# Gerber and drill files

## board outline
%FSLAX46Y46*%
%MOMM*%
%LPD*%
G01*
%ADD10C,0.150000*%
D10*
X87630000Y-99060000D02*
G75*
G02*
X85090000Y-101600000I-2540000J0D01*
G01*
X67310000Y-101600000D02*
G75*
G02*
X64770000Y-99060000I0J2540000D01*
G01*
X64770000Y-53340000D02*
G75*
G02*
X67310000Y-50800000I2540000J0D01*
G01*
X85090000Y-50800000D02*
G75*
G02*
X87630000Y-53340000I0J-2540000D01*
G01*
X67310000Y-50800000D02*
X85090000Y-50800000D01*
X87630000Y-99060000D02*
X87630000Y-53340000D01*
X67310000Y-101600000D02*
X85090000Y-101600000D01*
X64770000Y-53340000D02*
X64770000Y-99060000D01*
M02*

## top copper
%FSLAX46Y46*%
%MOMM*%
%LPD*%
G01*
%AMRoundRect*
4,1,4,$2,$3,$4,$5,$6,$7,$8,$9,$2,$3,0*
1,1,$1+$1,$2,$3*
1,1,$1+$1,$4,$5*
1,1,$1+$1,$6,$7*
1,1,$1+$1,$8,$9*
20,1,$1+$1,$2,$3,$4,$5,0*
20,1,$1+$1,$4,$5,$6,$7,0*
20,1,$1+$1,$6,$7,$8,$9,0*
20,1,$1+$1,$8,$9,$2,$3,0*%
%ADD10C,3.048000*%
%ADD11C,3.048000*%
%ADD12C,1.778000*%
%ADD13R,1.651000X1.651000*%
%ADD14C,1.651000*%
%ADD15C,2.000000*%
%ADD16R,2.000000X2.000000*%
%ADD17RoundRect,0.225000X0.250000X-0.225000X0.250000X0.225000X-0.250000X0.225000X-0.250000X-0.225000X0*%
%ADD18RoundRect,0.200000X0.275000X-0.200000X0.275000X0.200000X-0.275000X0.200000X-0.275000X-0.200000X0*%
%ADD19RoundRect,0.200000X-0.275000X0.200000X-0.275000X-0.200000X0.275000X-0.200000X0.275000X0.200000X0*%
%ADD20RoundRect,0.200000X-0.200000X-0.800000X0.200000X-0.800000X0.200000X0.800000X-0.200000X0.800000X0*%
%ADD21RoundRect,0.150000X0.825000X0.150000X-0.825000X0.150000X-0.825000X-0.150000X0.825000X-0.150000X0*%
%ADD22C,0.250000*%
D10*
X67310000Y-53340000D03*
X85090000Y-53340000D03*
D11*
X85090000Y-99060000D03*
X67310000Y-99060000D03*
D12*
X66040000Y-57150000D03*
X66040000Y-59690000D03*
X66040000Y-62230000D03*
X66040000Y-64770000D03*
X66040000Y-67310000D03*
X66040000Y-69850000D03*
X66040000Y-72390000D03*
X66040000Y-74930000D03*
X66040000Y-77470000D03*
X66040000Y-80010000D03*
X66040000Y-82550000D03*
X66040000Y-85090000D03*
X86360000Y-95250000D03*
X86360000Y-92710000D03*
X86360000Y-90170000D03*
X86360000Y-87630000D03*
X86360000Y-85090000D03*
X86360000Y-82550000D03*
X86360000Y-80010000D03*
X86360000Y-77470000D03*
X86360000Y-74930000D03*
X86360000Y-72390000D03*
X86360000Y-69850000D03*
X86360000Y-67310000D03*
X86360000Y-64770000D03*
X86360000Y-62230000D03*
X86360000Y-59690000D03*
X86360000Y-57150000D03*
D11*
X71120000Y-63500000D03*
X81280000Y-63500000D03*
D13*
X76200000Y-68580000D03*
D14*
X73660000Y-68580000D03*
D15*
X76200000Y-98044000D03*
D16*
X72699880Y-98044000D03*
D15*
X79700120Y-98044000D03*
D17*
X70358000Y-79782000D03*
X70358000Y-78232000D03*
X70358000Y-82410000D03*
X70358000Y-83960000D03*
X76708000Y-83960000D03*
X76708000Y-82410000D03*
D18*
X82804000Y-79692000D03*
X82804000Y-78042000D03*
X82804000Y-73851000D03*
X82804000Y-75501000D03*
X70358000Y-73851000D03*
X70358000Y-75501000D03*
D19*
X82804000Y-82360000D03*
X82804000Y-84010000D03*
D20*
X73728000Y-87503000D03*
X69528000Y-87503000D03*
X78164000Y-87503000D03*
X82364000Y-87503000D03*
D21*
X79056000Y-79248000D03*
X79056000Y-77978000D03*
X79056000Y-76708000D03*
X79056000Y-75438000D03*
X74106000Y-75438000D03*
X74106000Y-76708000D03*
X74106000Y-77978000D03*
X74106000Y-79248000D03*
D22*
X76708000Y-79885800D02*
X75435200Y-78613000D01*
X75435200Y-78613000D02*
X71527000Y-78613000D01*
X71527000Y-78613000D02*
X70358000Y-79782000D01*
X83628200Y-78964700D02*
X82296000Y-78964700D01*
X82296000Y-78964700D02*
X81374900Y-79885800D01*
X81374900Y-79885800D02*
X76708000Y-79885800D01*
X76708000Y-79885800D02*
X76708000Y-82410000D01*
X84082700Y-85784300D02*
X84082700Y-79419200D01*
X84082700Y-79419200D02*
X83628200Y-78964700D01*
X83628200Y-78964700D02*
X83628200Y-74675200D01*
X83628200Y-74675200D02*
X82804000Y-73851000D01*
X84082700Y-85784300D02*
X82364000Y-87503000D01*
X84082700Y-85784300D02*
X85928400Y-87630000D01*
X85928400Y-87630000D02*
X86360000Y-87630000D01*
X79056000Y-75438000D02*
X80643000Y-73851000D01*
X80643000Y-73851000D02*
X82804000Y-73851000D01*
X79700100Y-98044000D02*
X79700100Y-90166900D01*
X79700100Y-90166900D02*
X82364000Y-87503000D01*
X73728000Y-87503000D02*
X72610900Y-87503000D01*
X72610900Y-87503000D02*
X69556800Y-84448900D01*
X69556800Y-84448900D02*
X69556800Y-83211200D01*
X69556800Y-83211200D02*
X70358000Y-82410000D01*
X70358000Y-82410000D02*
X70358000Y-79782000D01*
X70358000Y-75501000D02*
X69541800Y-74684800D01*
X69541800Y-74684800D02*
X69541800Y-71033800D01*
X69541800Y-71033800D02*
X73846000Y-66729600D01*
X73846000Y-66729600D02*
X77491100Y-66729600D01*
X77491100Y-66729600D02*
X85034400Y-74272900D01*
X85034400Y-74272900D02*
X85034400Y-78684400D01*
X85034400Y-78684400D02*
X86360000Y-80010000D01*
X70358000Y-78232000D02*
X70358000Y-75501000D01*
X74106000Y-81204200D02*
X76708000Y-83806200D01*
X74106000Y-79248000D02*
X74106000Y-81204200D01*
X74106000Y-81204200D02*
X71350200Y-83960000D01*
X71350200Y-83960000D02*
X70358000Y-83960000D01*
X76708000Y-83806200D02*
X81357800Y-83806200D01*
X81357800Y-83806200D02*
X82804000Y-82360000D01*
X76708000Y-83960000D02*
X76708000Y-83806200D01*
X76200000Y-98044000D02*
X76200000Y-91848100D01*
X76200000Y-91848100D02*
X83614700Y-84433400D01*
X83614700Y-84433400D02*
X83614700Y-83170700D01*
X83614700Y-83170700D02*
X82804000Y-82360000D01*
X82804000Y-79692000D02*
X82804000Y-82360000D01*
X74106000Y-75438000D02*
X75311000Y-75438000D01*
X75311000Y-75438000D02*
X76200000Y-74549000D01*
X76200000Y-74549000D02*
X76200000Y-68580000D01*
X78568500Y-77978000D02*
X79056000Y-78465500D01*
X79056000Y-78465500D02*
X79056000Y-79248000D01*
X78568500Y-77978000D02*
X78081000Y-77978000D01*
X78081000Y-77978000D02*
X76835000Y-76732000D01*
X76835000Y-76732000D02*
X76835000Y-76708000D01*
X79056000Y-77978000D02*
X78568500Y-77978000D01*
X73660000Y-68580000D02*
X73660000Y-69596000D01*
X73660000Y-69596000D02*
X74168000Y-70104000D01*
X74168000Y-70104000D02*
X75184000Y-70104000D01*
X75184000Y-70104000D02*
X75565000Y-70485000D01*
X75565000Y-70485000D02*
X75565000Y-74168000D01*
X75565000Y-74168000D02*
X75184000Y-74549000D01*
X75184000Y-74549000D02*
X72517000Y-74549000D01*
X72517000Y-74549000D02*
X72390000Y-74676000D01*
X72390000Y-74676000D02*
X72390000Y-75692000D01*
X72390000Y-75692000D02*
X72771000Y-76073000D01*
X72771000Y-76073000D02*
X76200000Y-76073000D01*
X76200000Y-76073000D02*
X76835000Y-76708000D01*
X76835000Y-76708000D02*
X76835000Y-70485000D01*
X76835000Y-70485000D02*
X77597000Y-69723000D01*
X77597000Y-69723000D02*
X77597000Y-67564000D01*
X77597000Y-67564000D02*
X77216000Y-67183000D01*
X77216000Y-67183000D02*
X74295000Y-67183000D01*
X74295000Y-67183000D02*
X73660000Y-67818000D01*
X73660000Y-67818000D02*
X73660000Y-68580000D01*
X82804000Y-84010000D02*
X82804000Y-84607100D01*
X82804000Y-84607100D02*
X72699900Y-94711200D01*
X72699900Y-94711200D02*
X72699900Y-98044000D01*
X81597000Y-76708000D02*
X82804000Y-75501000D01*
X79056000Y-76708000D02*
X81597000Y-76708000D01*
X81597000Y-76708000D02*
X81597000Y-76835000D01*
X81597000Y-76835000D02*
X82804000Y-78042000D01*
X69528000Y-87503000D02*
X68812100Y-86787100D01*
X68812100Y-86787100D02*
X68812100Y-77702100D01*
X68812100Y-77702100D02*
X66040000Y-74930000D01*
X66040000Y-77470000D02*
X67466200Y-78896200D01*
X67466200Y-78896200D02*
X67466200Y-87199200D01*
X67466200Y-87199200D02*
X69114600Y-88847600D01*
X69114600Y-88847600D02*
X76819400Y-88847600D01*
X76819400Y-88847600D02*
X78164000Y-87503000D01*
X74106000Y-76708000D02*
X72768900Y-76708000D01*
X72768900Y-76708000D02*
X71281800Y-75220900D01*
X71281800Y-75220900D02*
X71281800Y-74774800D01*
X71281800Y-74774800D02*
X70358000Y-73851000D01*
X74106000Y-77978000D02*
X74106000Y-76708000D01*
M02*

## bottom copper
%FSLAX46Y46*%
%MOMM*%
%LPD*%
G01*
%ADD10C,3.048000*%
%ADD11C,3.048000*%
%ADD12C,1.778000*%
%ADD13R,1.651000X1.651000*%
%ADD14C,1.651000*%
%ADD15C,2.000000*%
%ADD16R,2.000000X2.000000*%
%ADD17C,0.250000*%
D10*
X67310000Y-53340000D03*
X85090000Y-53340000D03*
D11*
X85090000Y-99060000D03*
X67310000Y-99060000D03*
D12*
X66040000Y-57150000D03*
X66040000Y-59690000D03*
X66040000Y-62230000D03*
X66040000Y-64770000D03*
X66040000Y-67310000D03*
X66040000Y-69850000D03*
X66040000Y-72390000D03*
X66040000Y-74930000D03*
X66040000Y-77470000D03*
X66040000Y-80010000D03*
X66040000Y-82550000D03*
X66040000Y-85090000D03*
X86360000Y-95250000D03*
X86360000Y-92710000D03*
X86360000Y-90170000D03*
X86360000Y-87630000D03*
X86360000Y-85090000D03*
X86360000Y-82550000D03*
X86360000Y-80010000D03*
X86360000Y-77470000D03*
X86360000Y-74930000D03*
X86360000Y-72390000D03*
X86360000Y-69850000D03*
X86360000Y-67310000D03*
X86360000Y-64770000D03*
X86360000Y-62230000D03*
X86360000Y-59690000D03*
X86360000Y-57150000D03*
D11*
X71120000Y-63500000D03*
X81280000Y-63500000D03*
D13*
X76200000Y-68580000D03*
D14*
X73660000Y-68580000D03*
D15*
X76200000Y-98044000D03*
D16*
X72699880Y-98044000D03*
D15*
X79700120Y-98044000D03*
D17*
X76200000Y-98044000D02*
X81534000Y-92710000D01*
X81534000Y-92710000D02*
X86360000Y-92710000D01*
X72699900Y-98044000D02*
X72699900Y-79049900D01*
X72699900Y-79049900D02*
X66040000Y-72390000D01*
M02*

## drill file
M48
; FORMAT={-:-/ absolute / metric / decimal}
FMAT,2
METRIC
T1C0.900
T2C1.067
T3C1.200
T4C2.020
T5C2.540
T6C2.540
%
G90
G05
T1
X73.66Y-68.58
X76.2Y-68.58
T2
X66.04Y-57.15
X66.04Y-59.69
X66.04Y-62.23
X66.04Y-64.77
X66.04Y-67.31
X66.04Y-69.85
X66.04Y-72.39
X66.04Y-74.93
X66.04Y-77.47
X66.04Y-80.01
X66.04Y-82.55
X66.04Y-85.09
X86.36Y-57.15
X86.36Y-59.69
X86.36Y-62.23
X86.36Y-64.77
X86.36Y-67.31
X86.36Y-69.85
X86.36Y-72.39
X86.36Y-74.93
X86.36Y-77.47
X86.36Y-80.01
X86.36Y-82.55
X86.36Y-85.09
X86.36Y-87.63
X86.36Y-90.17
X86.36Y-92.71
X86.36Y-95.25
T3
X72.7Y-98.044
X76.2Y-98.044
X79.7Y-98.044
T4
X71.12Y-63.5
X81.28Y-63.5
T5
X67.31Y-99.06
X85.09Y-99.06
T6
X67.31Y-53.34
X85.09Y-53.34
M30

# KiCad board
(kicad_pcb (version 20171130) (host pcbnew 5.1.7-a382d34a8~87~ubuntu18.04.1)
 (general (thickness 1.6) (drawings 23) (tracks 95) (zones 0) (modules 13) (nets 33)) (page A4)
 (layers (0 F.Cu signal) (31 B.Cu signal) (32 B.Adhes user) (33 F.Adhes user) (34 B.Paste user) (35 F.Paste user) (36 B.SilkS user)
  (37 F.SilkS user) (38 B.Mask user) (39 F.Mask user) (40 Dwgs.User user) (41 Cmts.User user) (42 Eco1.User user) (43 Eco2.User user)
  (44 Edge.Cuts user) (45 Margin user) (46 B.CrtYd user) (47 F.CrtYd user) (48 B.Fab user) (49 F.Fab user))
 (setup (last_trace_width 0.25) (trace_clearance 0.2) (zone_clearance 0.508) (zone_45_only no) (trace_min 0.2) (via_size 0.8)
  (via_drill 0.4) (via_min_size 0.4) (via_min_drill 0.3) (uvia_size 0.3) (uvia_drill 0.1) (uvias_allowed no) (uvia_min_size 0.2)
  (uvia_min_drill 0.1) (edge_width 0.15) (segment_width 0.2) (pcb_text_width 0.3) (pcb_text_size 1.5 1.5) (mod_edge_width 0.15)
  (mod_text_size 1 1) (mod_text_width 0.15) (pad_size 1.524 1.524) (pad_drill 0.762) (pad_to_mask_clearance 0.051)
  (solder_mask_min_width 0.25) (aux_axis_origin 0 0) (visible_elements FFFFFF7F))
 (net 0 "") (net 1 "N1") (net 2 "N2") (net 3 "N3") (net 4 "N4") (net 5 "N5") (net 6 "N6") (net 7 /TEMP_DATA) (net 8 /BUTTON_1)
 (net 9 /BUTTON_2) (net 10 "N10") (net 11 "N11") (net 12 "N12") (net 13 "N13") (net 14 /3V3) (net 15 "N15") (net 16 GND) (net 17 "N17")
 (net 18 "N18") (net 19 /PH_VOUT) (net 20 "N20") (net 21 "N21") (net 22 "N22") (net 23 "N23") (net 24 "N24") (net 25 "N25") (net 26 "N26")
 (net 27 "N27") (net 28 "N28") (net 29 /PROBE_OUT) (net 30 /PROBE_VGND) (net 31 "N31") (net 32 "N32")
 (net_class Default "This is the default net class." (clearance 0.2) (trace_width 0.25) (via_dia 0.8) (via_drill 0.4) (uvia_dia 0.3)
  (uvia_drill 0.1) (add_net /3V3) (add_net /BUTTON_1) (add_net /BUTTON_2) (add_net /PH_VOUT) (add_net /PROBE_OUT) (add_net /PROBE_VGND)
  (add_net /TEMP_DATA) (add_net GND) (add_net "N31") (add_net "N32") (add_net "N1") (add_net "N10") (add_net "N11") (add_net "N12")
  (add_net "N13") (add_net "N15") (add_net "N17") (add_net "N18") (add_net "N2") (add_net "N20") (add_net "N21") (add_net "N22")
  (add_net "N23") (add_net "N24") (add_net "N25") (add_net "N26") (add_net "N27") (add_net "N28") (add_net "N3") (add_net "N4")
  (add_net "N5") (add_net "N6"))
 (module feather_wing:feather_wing (layer F.Cu) (at 76.2 76.2)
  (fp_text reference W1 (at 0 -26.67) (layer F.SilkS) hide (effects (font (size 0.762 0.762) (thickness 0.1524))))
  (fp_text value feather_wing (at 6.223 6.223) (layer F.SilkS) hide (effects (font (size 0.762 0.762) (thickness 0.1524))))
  (pad "" np_thru_hole circle (at -8.89 -22.86) (size 3.048 3.048) (drill 2.54) (layers *.Cu *.Mask))
  (pad "" np_thru_hole circle (at 8.89 -22.86) (size 3.048 3.048) (drill 2.54) (layers *.Cu *.Mask))
  (pad "" thru_hole circle (at 8.89 22.86) (size 3.048 3.048) (drill 2.54) (layers *.Cu *.Mask))
  (pad "" thru_hole circle (at -8.89 22.86) (size 3.048 3.048) (drill 2.54) (layers *.Cu *.Mask))
  (pad 1 thru_hole circle (at -10.16 -19.05) (size 1.778 1.778) (drill 1.0668) (layers *.Cu *.Mask) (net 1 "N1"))
  (pad 2 thru_hole circle (at -10.16 -16.51) (size 1.778 1.778) (drill 1.0668) (layers *.Cu *.Mask) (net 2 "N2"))
  (pad 3 thru_hole circle (at -10.16 -13.97) (size 1.778 1.778) (drill 1.0668) (layers *.Cu *.Mask) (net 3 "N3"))
  (pad 4 thru_hole circle (at -10.16 -11.43) (size 1.778 1.778) (drill 1.0668) (layers *.Cu *.Mask) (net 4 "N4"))
  (pad 5 thru_hole circle (at -10.16 -8.89) (size 1.778 1.778) (drill 1.0668) (layers *.Cu *.Mask) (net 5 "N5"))
  (pad 6 thru_hole circle (at -10.16 -6.35) (size 1.778 1.778) (drill 1.0668) (layers *.Cu *.Mask) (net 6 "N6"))
  (pad 7 thru_hole circle (at -10.16 -3.81) (size 1.778 1.778) (drill 1.0668) (layers *.Cu *.Mask) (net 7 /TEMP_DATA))
  (pad 8 thru_hole circle (at -10.16 -1.27) (size 1.778 1.778) (drill 1.0668) (layers *.Cu *.Mask) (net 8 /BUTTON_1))
  (pad 9 thru_hole circle (at -10.16 1.27) (size 1.778 1.778) (drill 1.0668) (layers *.Cu *.Mask) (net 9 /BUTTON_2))
  (pad 10 thru_hole circle (at -10.16 3.81) (size 1.778 1.778) (drill 1.0668) (layers *.Cu *.Mask) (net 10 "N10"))
  (pad 11 thru_hole circle (at -10.16 6.35) (size 1.778 1.778) (drill 1.0668) (layers *.Cu *.Mask) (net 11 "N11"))
  (pad 12 thru_hole circle (at -10.16 8.89) (size 1.778 1.778) (drill 1.0668) (layers *.Cu *.Mask) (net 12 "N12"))
  (pad 13 thru_hole circle (at 10.16 19.05) (size 1.778 1.778) (drill 1.0668) (layers *.Cu *.Mask) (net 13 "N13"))
  (pad 14 thru_hole circle (at 10.16 16.51) (size 1.778 1.778) (drill 1.0668) (layers *.Cu *.Mask) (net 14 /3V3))
  (pad 15 thru_hole circle (at 10.16 13.97) (size 1.778 1.778) (drill 1.0668) (layers *.Cu *.Mask) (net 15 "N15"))
  (pad 16 thru_hole circle (at 10.16 11.43) (size 1.778 1.778) (drill 1.0668) (layers *.Cu *.Mask) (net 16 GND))
  (pad 17 thru_hole circle (at 10.16 8.89) (size 1.778 1.778) (drill 1.0668) (layers *.Cu *.Mask) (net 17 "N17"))
  (pad 18 thru_hole circle (at 10.16 6.35) (size 1.778 1.778) (drill 1.0668) (layers *.Cu *.Mask) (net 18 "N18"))
  (pad 19 thru_hole circle (at 10.16 3.81) (size 1.778 1.778) (drill 1.0668) (layers *.Cu *.Mask) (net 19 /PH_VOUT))
  (pad 20 thru_hole circle (at 10.16 1.27) (size 1.778 1.778) (drill 1.0668) (layers *.Cu *.Mask) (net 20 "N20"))
  (pad 21 thru_hole circle (at 10.16 -1.27) (size 1.778 1.778) (drill 1.0668) (layers *.Cu *.Mask) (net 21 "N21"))
  (pad 22 thru_hole circle (at 10.16 -3.81) (size 1.778 1.778) (drill 1.0668) (layers *.Cu *.Mask) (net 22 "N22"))
  (pad 23 thru_hole circle (at 10.16 -6.35) (size 1.778 1.778) (drill 1.0668) (layers *.Cu *.Mask) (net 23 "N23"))
  (pad 24 thru_hole circle (at 10.16 -8.89) (size 1.778 1.778) (drill 1.0668) (layers *.Cu *.Mask) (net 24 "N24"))
  (pad 25 thru_hole circle (at 10.16 -11.43) (size 1.778 1.778) (drill 1.0668) (layers *.Cu *.Mask) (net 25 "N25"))
  (pad 26 thru_hole circle (at 10.16 -13.97) (size 1.778 1.778) (drill 1.0668) (layers *.Cu *.Mask) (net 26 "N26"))
  (pad 27 thru_hole circle (at 10.16 -16.51) (size 1.778 1.778) (drill 1.0668) (layers *.Cu *.Mask) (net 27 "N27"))
  (pad 28 thru_hole circle (at 10.16 -19.05) (size 1.778 1.778) (drill 1.0668) (layers *.Cu *.Mask) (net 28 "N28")))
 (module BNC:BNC (layer F.Cu) (at 76.2 63.5)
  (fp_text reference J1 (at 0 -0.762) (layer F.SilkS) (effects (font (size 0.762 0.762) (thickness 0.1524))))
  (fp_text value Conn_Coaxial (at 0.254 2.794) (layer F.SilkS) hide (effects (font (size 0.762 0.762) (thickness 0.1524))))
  (pad "" thru_hole circle (at -5.08 0) (size 3.048 3.048) (drill 2.02) (layers *.Cu *.Mask))
  (pad "" thru_hole circle (at 5.08 0) (size 3.048 3.048) (drill 2.02) (layers *.Cu *.Mask))
  (pad 1 thru_hole rect (at 0 5.08) (size 1.651 1.651) (drill 0.9) (layers *.Cu *.Mask) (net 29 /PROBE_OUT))
  (pad 2 thru_hole circle (at -2.54 5.08) (size 1.651 1.651) (drill 0.9) (layers *.Cu *.Mask) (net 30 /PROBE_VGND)))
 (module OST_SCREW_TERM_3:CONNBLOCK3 (layer F.Cu) (at 76.2 98.044)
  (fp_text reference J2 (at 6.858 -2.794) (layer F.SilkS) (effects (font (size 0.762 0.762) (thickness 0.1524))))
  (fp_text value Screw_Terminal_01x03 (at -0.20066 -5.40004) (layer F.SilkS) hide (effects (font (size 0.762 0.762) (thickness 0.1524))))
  (pad 2 thru_hole circle (at 0 0) (size 2 2) (drill 1.2) (layers *.Cu *.Mask) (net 14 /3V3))
  (pad 1 thru_hole rect (at -3.50012 0) (size 2 2) (drill 1.2) (layers *.Cu *.Mask) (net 7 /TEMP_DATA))
  (pad 3 thru_hole circle (at 3.50012 0) (size 2 2) (drill 1.2) (layers *.Cu *.Mask) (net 16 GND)))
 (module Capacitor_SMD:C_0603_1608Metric (layer F.Cu) (at 70.358 79.007 90)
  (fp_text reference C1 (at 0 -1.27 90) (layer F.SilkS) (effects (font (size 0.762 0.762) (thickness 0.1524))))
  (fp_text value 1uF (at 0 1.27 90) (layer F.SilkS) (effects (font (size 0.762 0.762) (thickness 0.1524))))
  (pad 1 smd roundrect (at -0.775 0 90) (size 0.9 0.95) (layers F.Cu F.Paste F.Mask) (roundrect_rratio 0.25) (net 16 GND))
  (pad 2 smd roundrect (at 0.775 0 90) (size 0.9 0.95) (layers F.Cu F.Paste F.Mask) (roundrect_rratio 0.25) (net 19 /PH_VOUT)))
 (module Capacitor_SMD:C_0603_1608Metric (layer F.Cu) (at 70.358 83.185 90)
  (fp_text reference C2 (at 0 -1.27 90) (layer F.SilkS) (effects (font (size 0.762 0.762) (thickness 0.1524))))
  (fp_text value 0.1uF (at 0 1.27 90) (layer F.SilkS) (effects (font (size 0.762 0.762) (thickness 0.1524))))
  (pad 2 smd roundrect (at 0.775 0 90) (size 0.9 0.95) (layers F.Cu F.Paste F.Mask) (roundrect_rratio 0.25) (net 16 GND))
  (pad 1 smd roundrect (at -0.775 0 90) (size 0.9 0.95) (layers F.Cu F.Paste F.Mask) (roundrect_rratio 0.25) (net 14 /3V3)))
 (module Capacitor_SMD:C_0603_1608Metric (layer F.Cu) (at 76.708 83.185 90)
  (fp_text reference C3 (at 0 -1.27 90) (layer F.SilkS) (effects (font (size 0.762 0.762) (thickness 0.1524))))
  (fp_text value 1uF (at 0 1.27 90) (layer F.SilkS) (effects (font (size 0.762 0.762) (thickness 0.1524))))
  (pad 1 smd roundrect (at -0.775 0 90) (size 0.9 0.95) (layers F.Cu F.Paste F.Mask) (roundrect_rratio 0.25) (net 14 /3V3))
  (pad 2 smd roundrect (at 0.775 0 90) (size 0.9 0.95) (layers F.Cu F.Paste F.Mask) (roundrect_rratio 0.25) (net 16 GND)))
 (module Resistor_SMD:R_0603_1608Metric (layer F.Cu) (at 82.804 78.867 90)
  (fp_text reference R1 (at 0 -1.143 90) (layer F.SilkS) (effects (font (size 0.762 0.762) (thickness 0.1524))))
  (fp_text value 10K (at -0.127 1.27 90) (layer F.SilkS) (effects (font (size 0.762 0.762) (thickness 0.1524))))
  (pad 1 smd roundrect (at -0.825 0 90) (size 0.8 0.95) (layers F.Cu F.Paste F.Mask) (roundrect_rratio 0.25) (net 14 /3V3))
  (pad 2 smd roundrect (at 0.825 0 90) (size 0.8 0.95) (layers F.Cu F.Paste F.Mask) (roundrect_rratio 0.25) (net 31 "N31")))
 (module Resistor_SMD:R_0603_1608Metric (layer F.Cu) (at 82.804 74.676 90)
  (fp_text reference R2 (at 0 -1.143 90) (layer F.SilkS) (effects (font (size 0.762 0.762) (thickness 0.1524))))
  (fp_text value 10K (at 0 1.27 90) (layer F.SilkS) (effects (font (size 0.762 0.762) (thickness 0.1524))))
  (pad 2 smd roundrect (at 0.825 0 90) (size 0.8 0.95) (layers F.Cu F.Paste F.Mask) (roundrect_rratio 0.25) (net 16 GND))
  (pad 1 smd roundrect (at -0.825 0 90) (size 0.8 0.95) (layers F.Cu F.Paste F.Mask) (roundrect_rratio 0.25) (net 31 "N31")))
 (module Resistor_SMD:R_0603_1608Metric (layer F.Cu) (at 70.358 74.676 90)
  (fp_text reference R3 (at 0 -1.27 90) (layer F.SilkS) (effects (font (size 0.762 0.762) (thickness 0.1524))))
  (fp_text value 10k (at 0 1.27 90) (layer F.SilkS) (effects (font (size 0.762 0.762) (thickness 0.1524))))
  (pad 2 smd roundrect (at 0.825 0 90) (size 0.8 0.95) (layers F.Cu F.Paste F.Mask) (roundrect_rratio 0.25) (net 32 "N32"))
  (pad 1 smd roundrect (at -0.825 0 90) (size 0.8 0.95) (layers F.Cu F.Paste F.Mask) (roundrect_rratio 0.25) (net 19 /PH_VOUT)))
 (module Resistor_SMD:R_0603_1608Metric (layer F.Cu) (at 82.804 83.185 270)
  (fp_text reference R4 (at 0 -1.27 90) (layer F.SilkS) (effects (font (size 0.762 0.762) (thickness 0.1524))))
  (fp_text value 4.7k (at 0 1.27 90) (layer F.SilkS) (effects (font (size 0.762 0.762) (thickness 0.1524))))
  (pad 1 smd roundrect (at -0.825 0 270) (size 0.8 0.95) (layers F.Cu F.Paste F.Mask) (roundrect_rratio 0.25) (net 14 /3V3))
  (pad 2 smd roundrect (at 0.825 0 270) (size 0.8 0.95) (layers F.Cu F.Paste F.Mask) (roundrect_rratio 0.25) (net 7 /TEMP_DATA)))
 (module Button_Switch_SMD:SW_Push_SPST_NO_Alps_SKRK (layer F.Cu) (at 71.628 87.503)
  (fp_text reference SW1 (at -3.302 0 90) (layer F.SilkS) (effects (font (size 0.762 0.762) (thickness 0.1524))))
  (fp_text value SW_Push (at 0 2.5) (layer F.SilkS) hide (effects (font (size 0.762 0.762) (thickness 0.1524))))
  (pad 2 smd roundrect (at 2.1 0) (size 0.8 2) (layers F.Cu F.Paste F.Mask) (roundrect_rratio 0.25) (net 16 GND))
  (pad 1 smd roundrect (at -2.1 0) (size 0.8 2) (layers F.Cu F.Paste F.Mask) (roundrect_rratio 0.25) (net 8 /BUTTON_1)))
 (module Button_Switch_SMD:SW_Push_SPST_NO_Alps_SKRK (layer F.Cu) (at 80.264 87.503)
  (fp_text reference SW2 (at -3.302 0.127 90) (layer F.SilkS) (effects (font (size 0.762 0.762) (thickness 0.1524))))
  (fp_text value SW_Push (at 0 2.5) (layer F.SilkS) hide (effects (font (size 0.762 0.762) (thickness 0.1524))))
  (pad 1 smd roundrect (at -2.1 0) (size 0.8 2) (layers F.Cu F.Paste F.Mask) (roundrect_rratio 0.25) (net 9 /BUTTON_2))
  (pad 2 smd roundrect (at 2.1 0) (size 0.8 2) (layers F.Cu F.Paste F.Mask) (roundrect_rratio 0.25) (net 16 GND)))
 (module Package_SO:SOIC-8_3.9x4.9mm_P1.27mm (layer F.Cu) (at 76.581 77.343 180)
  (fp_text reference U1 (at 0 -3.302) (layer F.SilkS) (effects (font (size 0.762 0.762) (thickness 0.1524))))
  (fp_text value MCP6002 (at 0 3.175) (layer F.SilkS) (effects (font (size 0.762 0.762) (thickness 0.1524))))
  (pad 1 smd roundrect (at -2.475 -1.905 180) (size 1.95 0.6) (layers F.Cu F.Paste F.Mask) (roundrect_rratio 0.25) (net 30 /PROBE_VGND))
  (pad 2 smd roundrect (at -2.475 -0.635 180) (size 1.95 0.6) (layers F.Cu F.Paste F.Mask) (roundrect_rratio 0.25) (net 30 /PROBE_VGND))
  (pad 3 smd roundrect (at -2.475 0.635 180) (size 1.95 0.6) (layers F.Cu F.Paste F.Mask) (roundrect_rratio 0.25) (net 31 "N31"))
  (pad 4 smd roundrect (at -2.475 1.905 180) (size 1.95 0.6) (layers F.Cu F.Paste F.Mask) (roundrect_rratio 0.25) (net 16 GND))
  (pad 5 smd roundrect (at 2.475 1.905 180) (size 1.95 0.6) (layers F.Cu F.Paste F.Mask) (roundrect_rratio 0.25) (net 29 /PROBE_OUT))
  (pad 6 smd roundrect (at 2.475 0.635 180) (size 1.95 0.6) (layers F.Cu F.Paste F.Mask) (roundrect_rratio 0.25) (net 32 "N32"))
  (pad 7 smd roundrect (at 2.475 -0.635 180) (size 1.95 0.6) (layers F.Cu F.Paste F.Mask) (roundrect_rratio 0.25) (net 32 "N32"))
  (pad 8 smd roundrect (at 2.475 -1.905 180) (size 1.95 0.6) (layers F.Cu F.Paste F.Mask) (roundrect_rratio 0.25) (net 14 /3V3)))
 (gr_arc (start 85.09 99.06) (end 85.09 101.6) (angle -90) (layer Edge.Cuts) (width 0.15))
 (gr_arc (start 67.31 99.06) (end 64.77 99.06) (angle -90) (layer Edge.Cuts) (width 0.15))
 (gr_arc (start 67.31 53.34) (end 67.31 50.8) (angle -90) (layer Edge.Cuts) (width 0.15))
 (gr_arc (start 85.09 53.34) (end 87.63 53.34) (angle -90) (layer Edge.Cuts) (width 0.15))
 (gr_line (start 67.31 50.8) (end 85.09 50.8) (layer Edge.Cuts) (width 0.15))
 (gr_line (start 87.63 99.06) (end 87.63 53.34) (layer Edge.Cuts) (width 0.15))
 (gr_line (start 67.31 101.6) (end 85.09 101.6) (layer Edge.Cuts) (width 0.15))
 (gr_line (start 64.77 53.34) (end 64.77 99.06) (layer Edge.Cuts) (width 0.15))
 (segment (start 76.708 79.8858) (end 75.4352 78.613) (width 0.25) (layer F.Cu) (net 16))
 (segment (start 75.4352 78.613) (end 71.527 78.613) (width 0.25) (layer F.Cu) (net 16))
 (segment (start 71.527 78.613) (end 70.358 79.782) (width 0.25) (layer F.Cu) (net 16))
 (segment (start 83.6282 78.9647) (end 82.296 78.9647) (width 0.25) (layer F.Cu) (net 16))
 (segment (start 82.296 78.9647) (end 81.3749 79.8858) (width 0.25) (layer F.Cu) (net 16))
 (segment (start 81.3749 79.8858) (end 76.708 79.8858) (width 0.25) (layer F.Cu) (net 16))
 (segment (start 76.708 79.8858) (end 76.708 82.41) (width 0.25) (layer F.Cu) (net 16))
 (segment (start 84.0827 85.7843) (end 84.0827 79.4192) (width 0.25) (layer F.Cu) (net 16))
 (segment (start 84.0827 79.4192) (end 83.6282 78.9647) (width 0.25) (layer F.Cu) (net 16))
 (segment (start 83.6282 78.9647) (end 83.6282 74.6752) (width 0.25) (layer F.Cu) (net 16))
 (segment (start 83.6282 74.6752) (end 82.804 73.851) (width 0.25) (layer F.Cu) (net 16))
 (segment (start 84.0827 85.7843) (end 82.364 87.503) (width 0.25) (layer F.Cu) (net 16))
 (segment (start 84.0827 85.7843) (end 85.9284 87.63) (width 0.25) (layer F.Cu) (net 16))
 (segment (start 85.9284 87.63) (end 86.36 87.63) (width 0.25) (layer F.Cu) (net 16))
 (segment (start 79.056 75.438) (end 80.643 73.851) (width 0.25) (layer F.Cu) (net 16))
 (segment (start 80.643 73.851) (end 82.804 73.851) (width 0.25) (layer F.Cu) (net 16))
 (segment (start 79.7001 98.044) (end 79.7001 90.1669) (width 0.25) (layer F.Cu) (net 16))
 (segment (start 79.7001 90.1669) (end 82.364 87.503) (width 0.25) (layer F.Cu) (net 16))
 (segment (start 73.728 87.503) (end 72.6109 87.503) (width 0.25) (layer F.Cu) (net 16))
 (segment (start 72.6109 87.503) (end 69.5568 84.4489) (width 0.25) (layer F.Cu) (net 16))
 (segment (start 69.5568 84.4489) (end 69.5568 83.2112) (width 0.25) (layer F.Cu) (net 16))
 (segment (start 69.5568 83.2112) (end 70.358 82.41) (width 0.25) (layer F.Cu) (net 16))
 (segment (start 70.358 82.41) (end 70.358 79.782) (width 0.25) (layer F.Cu) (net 16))
 (segment (start 70.358 75.501) (end 69.5418 74.6848) (width 0.25) (layer F.Cu) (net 19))
 (segment (start 69.5418 74.6848) (end 69.5418 71.0338) (width 0.25) (layer F.Cu) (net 19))
 (segment (start 69.5418 71.0338) (end 73.846 66.7296) (width 0.25) (layer F.Cu) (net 19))
 (segment (start 73.846 66.7296) (end 77.4911 66.7296) (width 0.25) (layer F.Cu) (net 19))
 (segment (start 77.4911 66.7296) (end 85.0344 74.2729) (width 0.25) (layer F.Cu) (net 19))
 (segment (start 85.0344 74.2729) (end 85.0344 78.6844) (width 0.25) (layer F.Cu) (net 19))
 (segment (start 85.0344 78.6844) (end 86.36 80.01) (width 0.25) (layer F.Cu) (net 19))
 (segment (start 70.358 78.232) (end 70.358 75.501) (width 0.25) (layer F.Cu) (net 19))
 (segment (start 74.106 81.2042) (end 76.708 83.8062) (width 0.25) (layer F.Cu) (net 14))
 (segment (start 74.106 79.248) (end 74.106 81.2042) (width 0.25) (layer F.Cu) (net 14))
 (segment (start 74.106 81.2042) (end 71.3502 83.96) (width 0.25) (layer F.Cu) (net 14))
 (segment (start 71.3502 83.96) (end 70.358 83.96) (width 0.25) (layer F.Cu) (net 14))
 (segment (start 76.708 83.8062) (end 81.3578 83.8062) (width 0.25) (layer F.Cu) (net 14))
 (segment (start 81.3578 83.8062) (end 82.804 82.36) (width 0.25) (layer F.Cu) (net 14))
 (segment (start 76.708 83.96) (end 76.708 83.8062) (width 0.25) (layer F.Cu) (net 14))
 (segment (start 76.2 98.044) (end 76.2 91.8481) (width 0.25) (layer F.Cu) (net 14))
 (segment (start 76.2 91.8481) (end 83.6147 84.4334) (width 0.25) (layer F.Cu) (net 14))
 (segment (start 83.6147 84.4334) (end 83.6147 83.1707) (width 0.25) (layer F.Cu) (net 14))
 (segment (start 83.6147 83.1707) (end 82.804 82.36) (width 0.25) (layer F.Cu) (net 14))
 (segment (start 82.804 79.692) (end 82.804 82.36) (width 0.25) (layer F.Cu) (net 14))
 (segment (start 76.2 98.044) (end 81.534 92.71) (width 0.25) (layer B.Cu) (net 14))
 (segment (start 81.534 92.71) (end 86.36 92.71) (width 0.25) (layer B.Cu) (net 14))
 (segment (start 74.106 75.438) (end 75.311 75.438) (width 0.25) (layer F.Cu) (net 29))
 (segment (start 75.311 75.438) (end 76.2 74.549) (width 0.25) (layer F.Cu) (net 29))
 (segment (start 76.2 74.549) (end 76.2 68.58) (width 0.25) (layer F.Cu) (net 29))
 (segment (start 78.5685 77.978) (end 79.056 78.4655) (width 0.25) (layer F.Cu) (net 30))
 (segment (start 79.056 78.4655) (end 79.056 79.248) (width 0.25) (layer F.Cu) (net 30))
 (segment (start 78.5685 77.978) (end 78.081 77.978) (width 0.25) (layer F.Cu) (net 30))
 (segment (start 78.081 77.978) (end 76.835 76.732) (width 0.25) (layer F.Cu) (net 30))
 (segment (start 76.835 76.732) (end 76.835 76.708) (width 0.25) (layer F.Cu) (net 30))
 (segment (start 79.056 77.978) (end 78.5685 77.978) (width 0.25) (layer F.Cu) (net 30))
 (segment (start 73.66 68.58) (end 73.66 69.596) (width 0.25) (layer F.Cu) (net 30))
 (segment (start 73.66 69.596) (end 74.168 70.104) (width 0.25) (layer F.Cu) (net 30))
 (segment (start 74.168 70.104) (end 75.184 70.104) (width 0.25) (layer F.Cu) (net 30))
 (segment (start 75.184 70.104) (end 75.565 70.485) (width 0.25) (layer F.Cu) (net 30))
 (segment (start 75.565 70.485) (end 75.565 74.168) (width 0.25) (layer F.Cu) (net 30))
 (segment (start 75.565 74.168) (end 75.184 74.549) (width 0.25) (layer F.Cu) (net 30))
 (segment (start 75.184 74.549) (end 72.517 74.549) (width 0.25) (layer F.Cu) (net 30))
 (segment (start 72.517 74.549) (end 72.39 74.676) (width 0.25) (layer F.Cu) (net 30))
 (segment (start 72.39 74.676) (end 72.39 75.692) (width 0.25) (layer F.Cu) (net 30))
 (segment (start 72.39 75.692) (end 72.771 76.073) (width 0.25) (layer F.Cu) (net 30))
 (segment (start 72.771 76.073) (end 76.2 76.073) (width 0.25) (layer F.Cu) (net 30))
 (segment (start 76.2 76.073) (end 76.835 76.708) (width 0.25) (layer F.Cu) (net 30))
 (segment (start 76.835 76.708) (end 76.835 70.485) (width 0.25) (layer F.Cu) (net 30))
 (segment (start 76.835 70.485) (end 77.597 69.723) (width 0.25) (layer F.Cu) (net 30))
 (segment (start 77.597 69.723) (end 77.597 67.564) (width 0.25) (layer F.Cu) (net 30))
 (segment (start 77.597 67.564) (end 77.216 67.183) (width 0.25) (layer F.Cu) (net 30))
 (segment (start 77.216 67.183) (end 74.295 67.183) (width 0.25) (layer F.Cu) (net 30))
 (segment (start 74.295 67.183) (end 73.66 67.818) (width 0.25) (layer F.Cu) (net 30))
 (segment (start 73.66 67.818) (end 73.66 68.58) (width 0.25) (layer F.Cu) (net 30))
 (segment (start 72.6999 98.044) (end 72.6999 79.0499) (width 0.25) (layer B.Cu) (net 7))
 (segment (start 72.6999 79.0499) (end 66.04 72.39) (width 0.25) (layer B.Cu) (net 7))
 (segment (start 82.804 84.01) (end 82.804 84.6071) (width 0.25) (layer F.Cu) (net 7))
 (segment (start 82.804 84.6071) (end 72.6999 94.7112) (width 0.25) (layer F.Cu) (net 7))
 (segment (start 72.6999 94.7112) (end 72.6999 98.044) (width 0.25) (layer F.Cu) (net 7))
 (segment (start 81.597 76.708) (end 82.804 75.501) (width 0.25) (layer F.Cu) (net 31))
 (segment (start 79.056 76.708) (end 81.597 76.708) (width 0.25) (layer F.Cu) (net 31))
 (segment (start 81.597 76.708) (end 81.597 76.835) (width 0.25) (layer F.Cu) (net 31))
 (segment (start 81.597 76.835) (end 82.804 78.042) (width 0.25) (layer F.Cu) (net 31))
 (segment (start 69.528 87.503) (end 68.8121 86.7871) (width 0.25) (layer F.Cu) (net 8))
 (segment (start 68.8121 86.7871) (end 68.8121 77.7021) (width 0.25) (layer F.Cu) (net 8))
 (segment (start 68.8121 77.7021) (end 66.04 74.93) (width 0.25) (layer F.Cu) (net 8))
 (segment (start 66.04 77.47) (end 67.4662 78.8962) (width 0.25) (layer F.Cu) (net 9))
 (segment (start 67.4662 78.8962) (end 67.4662 87.1992) (width 0.25) (layer F.Cu) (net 9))
 (segment (start 67.4662 87.1992) (end 69.1146 88.8476) (width 0.25) (layer F.Cu) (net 9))
 (segment (start 69.1146 88.8476) (end 76.8194 88.8476) (width 0.25) (layer F.Cu) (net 9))
 (segment (start 76.8194 88.8476) (end 78.164 87.503) (width 0.25) (layer F.Cu) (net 9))
 (segment (start 74.106 76.708) (end 72.7689 76.708) (width 0.25) (layer F.Cu) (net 32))
 (segment (start 72.7689 76.708) (end 71.2818 75.2209) (width 0.25) (layer F.Cu) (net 32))
 (segment (start 71.2818 75.2209) (end 71.2818 74.7748) (width 0.25) (layer F.Cu) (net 32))
 (segment (start 71.2818 74.7748) (end 70.358 73.851) (width 0.25) (layer F.Cu) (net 32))
 (segment (start 74.106 77.978) (end 74.106 76.708) (width 0.25) (layer F.Cu) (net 32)))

